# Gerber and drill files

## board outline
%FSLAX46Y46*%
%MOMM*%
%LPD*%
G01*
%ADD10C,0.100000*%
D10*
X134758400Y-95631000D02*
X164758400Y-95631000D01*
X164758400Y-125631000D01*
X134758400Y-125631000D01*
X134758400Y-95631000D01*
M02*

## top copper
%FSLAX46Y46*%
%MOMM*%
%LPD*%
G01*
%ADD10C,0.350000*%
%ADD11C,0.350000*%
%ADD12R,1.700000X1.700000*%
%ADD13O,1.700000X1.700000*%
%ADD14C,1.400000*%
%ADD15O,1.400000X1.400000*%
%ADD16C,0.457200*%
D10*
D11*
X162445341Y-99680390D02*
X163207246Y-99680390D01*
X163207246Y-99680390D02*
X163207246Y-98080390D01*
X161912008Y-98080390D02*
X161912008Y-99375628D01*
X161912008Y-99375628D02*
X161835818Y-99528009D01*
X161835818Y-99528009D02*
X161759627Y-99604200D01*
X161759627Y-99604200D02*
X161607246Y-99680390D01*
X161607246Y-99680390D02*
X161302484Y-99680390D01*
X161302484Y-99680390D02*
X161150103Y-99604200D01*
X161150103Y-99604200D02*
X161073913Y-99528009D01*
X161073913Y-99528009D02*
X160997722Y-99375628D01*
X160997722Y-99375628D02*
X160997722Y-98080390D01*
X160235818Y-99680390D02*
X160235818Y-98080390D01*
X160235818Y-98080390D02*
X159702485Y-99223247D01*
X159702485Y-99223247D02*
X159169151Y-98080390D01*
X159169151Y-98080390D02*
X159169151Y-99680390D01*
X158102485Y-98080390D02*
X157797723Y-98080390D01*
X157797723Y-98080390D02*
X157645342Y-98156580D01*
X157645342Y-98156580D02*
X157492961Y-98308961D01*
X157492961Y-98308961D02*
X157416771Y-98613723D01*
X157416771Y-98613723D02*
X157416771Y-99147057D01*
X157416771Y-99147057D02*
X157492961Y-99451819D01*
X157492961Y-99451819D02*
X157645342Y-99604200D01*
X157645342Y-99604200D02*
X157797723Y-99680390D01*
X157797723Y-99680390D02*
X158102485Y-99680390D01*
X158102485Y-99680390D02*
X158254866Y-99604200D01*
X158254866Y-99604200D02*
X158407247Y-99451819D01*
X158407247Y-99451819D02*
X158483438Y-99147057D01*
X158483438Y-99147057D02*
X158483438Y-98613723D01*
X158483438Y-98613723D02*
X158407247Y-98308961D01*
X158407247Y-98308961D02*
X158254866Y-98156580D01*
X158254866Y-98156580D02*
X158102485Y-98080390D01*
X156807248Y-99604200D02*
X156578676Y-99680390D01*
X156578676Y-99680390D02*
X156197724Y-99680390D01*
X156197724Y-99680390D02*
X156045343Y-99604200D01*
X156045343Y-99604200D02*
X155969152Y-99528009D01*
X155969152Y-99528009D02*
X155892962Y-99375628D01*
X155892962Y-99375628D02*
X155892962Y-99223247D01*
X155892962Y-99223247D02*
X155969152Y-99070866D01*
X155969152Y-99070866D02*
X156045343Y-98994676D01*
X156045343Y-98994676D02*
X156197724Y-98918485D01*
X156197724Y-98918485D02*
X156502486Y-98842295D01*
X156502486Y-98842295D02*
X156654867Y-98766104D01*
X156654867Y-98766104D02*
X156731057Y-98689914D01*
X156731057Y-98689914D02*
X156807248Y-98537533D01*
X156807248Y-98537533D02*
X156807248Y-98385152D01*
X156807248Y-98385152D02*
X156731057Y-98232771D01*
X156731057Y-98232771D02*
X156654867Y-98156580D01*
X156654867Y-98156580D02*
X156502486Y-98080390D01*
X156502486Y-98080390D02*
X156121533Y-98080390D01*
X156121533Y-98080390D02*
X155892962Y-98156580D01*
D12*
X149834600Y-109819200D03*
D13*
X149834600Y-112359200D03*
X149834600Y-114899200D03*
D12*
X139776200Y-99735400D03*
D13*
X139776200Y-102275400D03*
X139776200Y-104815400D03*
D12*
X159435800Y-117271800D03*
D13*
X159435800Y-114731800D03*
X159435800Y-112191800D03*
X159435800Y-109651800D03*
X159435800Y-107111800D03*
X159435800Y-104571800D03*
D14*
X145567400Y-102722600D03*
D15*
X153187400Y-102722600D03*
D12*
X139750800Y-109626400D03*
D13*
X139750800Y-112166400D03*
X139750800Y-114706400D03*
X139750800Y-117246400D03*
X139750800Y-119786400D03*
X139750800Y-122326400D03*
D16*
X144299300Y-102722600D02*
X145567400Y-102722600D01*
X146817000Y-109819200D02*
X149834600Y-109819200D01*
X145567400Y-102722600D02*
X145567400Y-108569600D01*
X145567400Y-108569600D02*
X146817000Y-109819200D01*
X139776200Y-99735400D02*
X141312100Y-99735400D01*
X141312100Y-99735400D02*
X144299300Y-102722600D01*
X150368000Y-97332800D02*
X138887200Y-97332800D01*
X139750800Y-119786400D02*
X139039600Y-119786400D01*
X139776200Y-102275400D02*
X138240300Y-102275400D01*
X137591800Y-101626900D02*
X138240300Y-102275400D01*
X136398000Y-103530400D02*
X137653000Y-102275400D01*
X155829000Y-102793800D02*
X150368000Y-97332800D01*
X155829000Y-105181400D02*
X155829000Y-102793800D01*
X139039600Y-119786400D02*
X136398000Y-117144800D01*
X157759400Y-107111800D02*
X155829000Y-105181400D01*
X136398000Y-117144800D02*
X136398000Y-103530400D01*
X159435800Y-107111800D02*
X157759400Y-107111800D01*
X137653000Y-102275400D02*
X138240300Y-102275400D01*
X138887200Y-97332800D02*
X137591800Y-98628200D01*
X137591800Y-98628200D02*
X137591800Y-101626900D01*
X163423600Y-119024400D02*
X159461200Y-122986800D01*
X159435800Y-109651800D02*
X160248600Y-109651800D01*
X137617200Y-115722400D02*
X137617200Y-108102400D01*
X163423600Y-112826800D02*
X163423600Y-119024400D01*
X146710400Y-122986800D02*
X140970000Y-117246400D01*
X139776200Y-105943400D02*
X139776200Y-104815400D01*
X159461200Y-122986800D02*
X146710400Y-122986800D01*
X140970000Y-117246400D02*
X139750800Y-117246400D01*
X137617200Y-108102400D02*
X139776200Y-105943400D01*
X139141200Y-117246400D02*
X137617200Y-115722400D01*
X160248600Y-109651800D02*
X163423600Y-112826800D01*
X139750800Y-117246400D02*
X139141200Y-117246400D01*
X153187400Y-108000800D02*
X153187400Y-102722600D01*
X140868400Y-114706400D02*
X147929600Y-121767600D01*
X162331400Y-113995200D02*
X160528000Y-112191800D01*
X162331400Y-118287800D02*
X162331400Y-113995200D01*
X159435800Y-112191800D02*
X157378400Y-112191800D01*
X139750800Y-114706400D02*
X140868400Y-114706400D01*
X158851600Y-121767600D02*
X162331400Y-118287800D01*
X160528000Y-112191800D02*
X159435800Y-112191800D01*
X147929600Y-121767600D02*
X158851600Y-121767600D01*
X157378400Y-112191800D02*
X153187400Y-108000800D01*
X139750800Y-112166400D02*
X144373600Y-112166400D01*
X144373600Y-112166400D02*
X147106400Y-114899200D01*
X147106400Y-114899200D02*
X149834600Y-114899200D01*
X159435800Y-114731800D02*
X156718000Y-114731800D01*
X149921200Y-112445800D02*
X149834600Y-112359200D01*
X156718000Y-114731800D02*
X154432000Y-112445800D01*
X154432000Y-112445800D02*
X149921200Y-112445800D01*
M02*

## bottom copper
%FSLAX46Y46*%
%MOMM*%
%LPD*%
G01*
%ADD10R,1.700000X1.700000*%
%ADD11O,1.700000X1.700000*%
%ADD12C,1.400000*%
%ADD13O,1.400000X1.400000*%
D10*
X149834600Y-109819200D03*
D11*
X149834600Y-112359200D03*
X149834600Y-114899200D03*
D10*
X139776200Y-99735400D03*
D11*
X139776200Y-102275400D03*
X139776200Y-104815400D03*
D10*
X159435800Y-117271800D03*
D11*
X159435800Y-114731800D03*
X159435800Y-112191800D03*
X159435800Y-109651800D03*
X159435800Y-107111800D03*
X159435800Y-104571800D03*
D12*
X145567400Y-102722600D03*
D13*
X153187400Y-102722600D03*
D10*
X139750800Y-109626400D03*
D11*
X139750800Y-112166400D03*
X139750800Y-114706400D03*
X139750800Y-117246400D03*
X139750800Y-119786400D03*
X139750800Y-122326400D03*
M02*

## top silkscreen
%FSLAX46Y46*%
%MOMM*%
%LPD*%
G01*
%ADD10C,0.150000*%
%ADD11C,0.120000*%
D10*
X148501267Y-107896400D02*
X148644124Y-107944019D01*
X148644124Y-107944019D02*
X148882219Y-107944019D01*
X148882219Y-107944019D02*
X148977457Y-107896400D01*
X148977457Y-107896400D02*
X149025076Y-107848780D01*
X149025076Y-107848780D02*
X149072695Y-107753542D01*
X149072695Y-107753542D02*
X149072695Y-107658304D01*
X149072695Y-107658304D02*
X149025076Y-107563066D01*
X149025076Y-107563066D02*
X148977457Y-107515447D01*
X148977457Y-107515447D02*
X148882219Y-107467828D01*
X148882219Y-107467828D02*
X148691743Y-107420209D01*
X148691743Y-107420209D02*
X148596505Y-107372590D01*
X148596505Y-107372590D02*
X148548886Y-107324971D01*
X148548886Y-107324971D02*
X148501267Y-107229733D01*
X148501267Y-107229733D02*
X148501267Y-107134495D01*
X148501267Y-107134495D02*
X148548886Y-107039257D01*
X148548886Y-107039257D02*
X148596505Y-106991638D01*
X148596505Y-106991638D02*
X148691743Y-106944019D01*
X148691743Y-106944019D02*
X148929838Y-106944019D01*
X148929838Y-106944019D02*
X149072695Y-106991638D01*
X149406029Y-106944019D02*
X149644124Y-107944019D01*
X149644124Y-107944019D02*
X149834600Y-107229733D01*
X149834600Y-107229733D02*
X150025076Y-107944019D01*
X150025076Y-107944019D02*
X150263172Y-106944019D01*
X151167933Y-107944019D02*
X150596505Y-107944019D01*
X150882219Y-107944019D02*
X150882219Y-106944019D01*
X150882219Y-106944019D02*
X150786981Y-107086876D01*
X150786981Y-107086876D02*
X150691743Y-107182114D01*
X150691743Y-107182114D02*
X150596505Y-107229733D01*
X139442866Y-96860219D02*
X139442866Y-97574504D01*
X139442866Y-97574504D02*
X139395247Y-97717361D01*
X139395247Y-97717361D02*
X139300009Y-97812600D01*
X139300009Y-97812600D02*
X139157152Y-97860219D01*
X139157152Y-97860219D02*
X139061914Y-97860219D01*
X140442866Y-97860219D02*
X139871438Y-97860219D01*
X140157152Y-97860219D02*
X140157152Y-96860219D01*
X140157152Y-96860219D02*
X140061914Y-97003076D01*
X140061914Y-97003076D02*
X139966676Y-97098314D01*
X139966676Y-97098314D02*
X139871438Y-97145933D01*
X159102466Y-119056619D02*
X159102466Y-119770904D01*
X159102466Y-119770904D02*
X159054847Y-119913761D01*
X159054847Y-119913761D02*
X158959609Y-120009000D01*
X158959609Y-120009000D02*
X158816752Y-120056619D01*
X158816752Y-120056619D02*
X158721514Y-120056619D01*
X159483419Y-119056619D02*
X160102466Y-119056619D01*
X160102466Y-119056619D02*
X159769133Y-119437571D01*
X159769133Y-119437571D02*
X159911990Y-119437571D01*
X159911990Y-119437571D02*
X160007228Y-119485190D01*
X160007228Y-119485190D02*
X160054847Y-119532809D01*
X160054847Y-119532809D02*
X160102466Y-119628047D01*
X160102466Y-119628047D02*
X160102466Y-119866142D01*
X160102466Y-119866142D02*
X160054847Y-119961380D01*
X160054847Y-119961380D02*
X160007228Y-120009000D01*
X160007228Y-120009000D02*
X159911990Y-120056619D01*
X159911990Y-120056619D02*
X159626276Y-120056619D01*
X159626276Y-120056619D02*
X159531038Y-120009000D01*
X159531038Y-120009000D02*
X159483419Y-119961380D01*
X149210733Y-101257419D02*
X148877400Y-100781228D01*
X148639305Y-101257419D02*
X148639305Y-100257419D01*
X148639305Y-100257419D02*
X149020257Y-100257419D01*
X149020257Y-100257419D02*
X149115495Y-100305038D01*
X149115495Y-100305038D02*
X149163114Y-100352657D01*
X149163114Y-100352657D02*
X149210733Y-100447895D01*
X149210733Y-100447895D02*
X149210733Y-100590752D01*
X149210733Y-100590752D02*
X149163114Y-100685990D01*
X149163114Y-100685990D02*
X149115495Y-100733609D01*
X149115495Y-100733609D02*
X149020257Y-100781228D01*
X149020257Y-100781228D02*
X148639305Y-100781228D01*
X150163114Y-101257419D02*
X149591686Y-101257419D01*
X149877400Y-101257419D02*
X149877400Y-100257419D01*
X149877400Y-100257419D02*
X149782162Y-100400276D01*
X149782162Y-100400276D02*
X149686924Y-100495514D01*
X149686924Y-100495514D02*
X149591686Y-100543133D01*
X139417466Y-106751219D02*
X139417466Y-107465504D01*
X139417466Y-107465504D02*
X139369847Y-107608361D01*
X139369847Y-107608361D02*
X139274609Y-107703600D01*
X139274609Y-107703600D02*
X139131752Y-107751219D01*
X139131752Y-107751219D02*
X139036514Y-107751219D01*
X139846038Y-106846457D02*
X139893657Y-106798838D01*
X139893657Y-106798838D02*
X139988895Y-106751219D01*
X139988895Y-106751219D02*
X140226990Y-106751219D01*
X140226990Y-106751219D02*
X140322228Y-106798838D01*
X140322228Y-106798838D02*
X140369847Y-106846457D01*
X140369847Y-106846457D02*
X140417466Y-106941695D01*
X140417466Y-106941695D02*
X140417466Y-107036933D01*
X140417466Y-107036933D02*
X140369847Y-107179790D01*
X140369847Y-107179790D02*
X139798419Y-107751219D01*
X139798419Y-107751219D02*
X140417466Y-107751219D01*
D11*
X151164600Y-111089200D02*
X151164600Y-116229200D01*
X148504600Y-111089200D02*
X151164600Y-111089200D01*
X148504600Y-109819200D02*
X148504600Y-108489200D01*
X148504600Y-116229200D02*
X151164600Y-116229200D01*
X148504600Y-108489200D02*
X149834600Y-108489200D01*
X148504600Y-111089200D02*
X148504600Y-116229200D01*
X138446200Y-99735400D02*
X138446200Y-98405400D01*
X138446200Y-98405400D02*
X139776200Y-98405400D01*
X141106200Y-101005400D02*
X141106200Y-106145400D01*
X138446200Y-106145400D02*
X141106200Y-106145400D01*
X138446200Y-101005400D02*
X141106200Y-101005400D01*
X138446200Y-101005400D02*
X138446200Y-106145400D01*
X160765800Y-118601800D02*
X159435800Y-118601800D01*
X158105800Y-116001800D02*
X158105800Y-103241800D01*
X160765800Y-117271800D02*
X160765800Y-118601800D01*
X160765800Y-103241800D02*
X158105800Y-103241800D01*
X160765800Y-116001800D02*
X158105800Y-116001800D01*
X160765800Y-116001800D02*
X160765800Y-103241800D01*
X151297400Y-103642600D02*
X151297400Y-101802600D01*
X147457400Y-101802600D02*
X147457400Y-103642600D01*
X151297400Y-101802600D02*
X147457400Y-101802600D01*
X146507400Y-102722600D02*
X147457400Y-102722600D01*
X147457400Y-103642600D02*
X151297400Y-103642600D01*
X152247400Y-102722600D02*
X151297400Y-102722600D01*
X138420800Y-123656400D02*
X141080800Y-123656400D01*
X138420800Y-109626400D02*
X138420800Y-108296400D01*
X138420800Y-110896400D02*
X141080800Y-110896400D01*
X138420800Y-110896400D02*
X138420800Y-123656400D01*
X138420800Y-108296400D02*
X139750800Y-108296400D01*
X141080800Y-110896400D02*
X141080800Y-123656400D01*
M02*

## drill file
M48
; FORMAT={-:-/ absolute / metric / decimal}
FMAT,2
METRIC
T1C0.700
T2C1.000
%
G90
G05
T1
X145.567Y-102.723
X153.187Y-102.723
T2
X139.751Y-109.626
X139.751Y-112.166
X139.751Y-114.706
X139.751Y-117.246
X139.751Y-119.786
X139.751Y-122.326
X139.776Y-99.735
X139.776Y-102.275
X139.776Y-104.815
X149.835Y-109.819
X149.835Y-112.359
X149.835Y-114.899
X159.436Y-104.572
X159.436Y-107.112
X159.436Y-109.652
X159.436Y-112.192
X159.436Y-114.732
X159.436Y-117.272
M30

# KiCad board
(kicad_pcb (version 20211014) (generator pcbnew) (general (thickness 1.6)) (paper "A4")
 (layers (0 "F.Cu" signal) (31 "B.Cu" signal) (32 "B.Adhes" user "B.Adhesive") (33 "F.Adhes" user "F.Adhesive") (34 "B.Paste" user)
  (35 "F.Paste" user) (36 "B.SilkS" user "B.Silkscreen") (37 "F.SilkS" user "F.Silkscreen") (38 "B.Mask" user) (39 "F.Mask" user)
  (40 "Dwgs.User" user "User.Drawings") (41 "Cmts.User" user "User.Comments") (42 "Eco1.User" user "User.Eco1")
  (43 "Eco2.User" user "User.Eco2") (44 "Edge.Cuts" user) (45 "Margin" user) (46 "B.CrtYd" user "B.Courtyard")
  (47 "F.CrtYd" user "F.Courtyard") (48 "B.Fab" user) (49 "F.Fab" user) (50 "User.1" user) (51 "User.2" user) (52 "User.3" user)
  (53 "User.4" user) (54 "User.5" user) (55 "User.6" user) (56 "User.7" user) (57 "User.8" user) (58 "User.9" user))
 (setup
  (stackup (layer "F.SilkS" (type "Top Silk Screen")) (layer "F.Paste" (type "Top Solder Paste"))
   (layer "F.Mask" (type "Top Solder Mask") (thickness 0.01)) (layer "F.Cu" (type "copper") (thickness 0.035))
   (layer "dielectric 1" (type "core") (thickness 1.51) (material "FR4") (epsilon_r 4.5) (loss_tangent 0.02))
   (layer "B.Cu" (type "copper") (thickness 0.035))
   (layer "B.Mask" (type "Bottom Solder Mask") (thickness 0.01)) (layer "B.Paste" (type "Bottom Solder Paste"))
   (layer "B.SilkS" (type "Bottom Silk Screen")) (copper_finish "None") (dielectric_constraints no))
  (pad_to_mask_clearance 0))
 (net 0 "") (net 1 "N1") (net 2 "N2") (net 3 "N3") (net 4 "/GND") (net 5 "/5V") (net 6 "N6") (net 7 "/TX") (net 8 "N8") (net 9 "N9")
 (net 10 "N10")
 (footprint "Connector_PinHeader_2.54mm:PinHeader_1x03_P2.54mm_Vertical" (layer "F.Cu") (at 149.8346 109.8192)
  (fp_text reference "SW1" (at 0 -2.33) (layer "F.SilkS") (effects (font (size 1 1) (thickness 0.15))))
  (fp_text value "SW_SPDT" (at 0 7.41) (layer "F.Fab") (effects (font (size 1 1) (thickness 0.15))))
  (fp_line (start 1.33 1.27) (end 1.33 6.41) (layer "F.SilkS") (width 0.12))
  (fp_line (start -1.33 1.27) (end 1.33 1.27) (layer "F.SilkS") (width 0.12))
  (fp_line (start -1.33 0) (end -1.33 -1.33) (layer "F.SilkS") (width 0.12))
  (fp_line (start -1.33 6.41) (end 1.33 6.41) (layer "F.SilkS") (width 0.12))
  (fp_line (start -1.33 -1.33) (end 0 -1.33) (layer "F.SilkS") (width 0.12))
  (fp_line (start -1.33 1.27) (end -1.33 6.41) (layer "F.SilkS") (width 0.12))
  (pad "1" thru_hole rect (at 0 0) (size 1.7 1.7) (drill 1) (layers *.Cu *.Mask) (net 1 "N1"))
  (pad "2" thru_hole oval (at 0 2.54) (size 1.7 1.7) (drill 1) (layers *.Cu *.Mask) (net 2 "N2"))
  (pad "3" thru_hole oval (at 0 5.08) (size 1.7 1.7) (drill 1) (layers *.Cu *.Mask) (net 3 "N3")))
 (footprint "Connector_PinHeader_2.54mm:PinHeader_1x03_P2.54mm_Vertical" (layer "F.Cu") (at 139.7762 99.7354)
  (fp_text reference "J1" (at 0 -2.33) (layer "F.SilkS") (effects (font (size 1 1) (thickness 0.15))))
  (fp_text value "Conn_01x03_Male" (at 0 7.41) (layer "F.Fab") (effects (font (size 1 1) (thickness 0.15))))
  (fp_line (start -1.33 0) (end -1.33 -1.33) (layer "F.SilkS") (width 0.12))
  (fp_line (start -1.33 -1.33) (end 0 -1.33) (layer "F.SilkS") (width 0.12))
  (fp_line (start 1.33 1.27) (end 1.33 6.41) (layer "F.SilkS") (width 0.12))
  (fp_line (start -1.33 6.41) (end 1.33 6.41) (layer "F.SilkS") (width 0.12))
  (fp_line (start -1.33 1.27) (end 1.33 1.27) (layer "F.SilkS") (width 0.12))
  (fp_line (start -1.33 1.27) (end -1.33 6.41) (layer "F.SilkS") (width 0.12))
  (pad "1" thru_hole rect (at 0 0) (size 1.7 1.7) (drill 1) (layers *.Cu *.Mask) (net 1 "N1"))
  (pad "2" thru_hole oval (at 0 2.54) (size 1.7 1.7) (drill 1) (layers *.Cu *.Mask) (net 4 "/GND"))
  (pad "3" thru_hole oval (at 0 5.08) (size 1.7 1.7) (drill 1) (layers *.Cu *.Mask) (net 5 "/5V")))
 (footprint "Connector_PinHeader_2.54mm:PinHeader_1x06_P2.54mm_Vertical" (layer "F.Cu") (at 159.4358 117.2718 180)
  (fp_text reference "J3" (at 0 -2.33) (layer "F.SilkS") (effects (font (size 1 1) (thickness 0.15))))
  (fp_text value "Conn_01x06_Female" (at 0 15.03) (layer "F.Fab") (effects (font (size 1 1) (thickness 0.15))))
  (fp_line (start -1.33 -1.33) (end 0 -1.33) (layer "F.SilkS") (width 0.12))
  (fp_line (start 1.33 1.27) (end 1.33 14.03) (layer "F.SilkS") (width 0.12))
  (fp_line (start -1.33 0) (end -1.33 -1.33) (layer "F.SilkS") (width 0.12))
  (fp_line (start -1.33 14.03) (end 1.33 14.03) (layer "F.SilkS") (width 0.12))
  (fp_line (start -1.33 1.27) (end 1.33 1.27) (layer "F.SilkS") (width 0.12))
  (fp_line (start -1.33 1.27) (end -1.33 14.03) (layer "F.SilkS") (width 0.12))
  (pad "1" thru_hole rect (at 0 0 180) (size 1.7 1.7) (drill 1) (layers *.Cu *.Mask) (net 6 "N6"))
  (pad "2" thru_hole oval (at 0 2.54 180) (size 1.7 1.7) (drill 1) (layers *.Cu *.Mask) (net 2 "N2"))
  (pad "3" thru_hole oval (at 0 5.08 180) (size 1.7 1.7) (drill 1) (layers *.Cu *.Mask) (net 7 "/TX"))
  (pad "4" thru_hole oval (at 0 7.62 180) (size 1.7 1.7) (drill 1) (layers *.Cu *.Mask) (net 5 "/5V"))
  (pad "5" thru_hole oval (at 0 10.16 180) (size 1.7 1.7) (drill 1) (layers *.Cu *.Mask) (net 4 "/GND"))
  (pad "6" thru_hole oval (at 0 12.7 180) (size 1.7 1.7) (drill 1) (layers *.Cu *.Mask) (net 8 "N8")))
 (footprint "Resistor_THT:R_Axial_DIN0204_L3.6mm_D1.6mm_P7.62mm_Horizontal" (layer "F.Cu") (at 145.5674 102.7226)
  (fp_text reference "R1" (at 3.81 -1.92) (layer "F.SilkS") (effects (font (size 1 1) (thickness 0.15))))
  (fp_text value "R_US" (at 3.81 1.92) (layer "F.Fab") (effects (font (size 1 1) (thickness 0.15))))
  (fp_line (start 5.73 0.92) (end 5.73 -0.92) (layer "F.SilkS") (width 0.12))
  (fp_line (start 1.89 -0.92) (end 1.89 0.92) (layer "F.SilkS") (width 0.12))
  (fp_line (start 5.73 -0.92) (end 1.89 -0.92) (layer "F.SilkS") (width 0.12))
  (fp_line (start 0.94 0) (end 1.89 0) (layer "F.SilkS") (width 0.12))
  (fp_line (start 1.89 0.92) (end 5.73 0.92) (layer "F.SilkS") (width 0.12))
  (fp_line (start 6.68 0) (end 5.73 0) (layer "F.SilkS") (width 0.12))
  (pad "1" thru_hole circle (at 0 0) (size 1.4 1.4) (drill 0.7) (layers *.Cu *.Mask) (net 1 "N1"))
  (pad "2" thru_hole oval (at 7.62 0) (size 1.4 1.4) (drill 0.7) (layers *.Cu *.Mask) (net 7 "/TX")))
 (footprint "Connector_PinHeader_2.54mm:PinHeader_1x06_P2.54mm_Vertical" (layer "F.Cu") (at 139.7508 109.6264)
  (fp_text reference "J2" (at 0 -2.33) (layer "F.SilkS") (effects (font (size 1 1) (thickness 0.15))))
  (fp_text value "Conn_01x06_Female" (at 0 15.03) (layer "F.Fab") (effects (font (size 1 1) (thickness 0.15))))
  (fp_line (start -1.33 14.03) (end 1.33 14.03) (layer "F.SilkS") (width 0.12))
  (fp_line (start -1.33 0) (end -1.33 -1.33) (layer "F.SilkS") (width 0.12))
  (fp_line (start -1.33 1.27) (end 1.33 1.27) (layer "F.SilkS") (width 0.12))
  (fp_line (start -1.33 1.27) (end -1.33 14.03) (layer "F.SilkS") (width 0.12))
  (fp_line (start -1.33 -1.33) (end 0 -1.33) (layer "F.SilkS") (width 0.12))
  (fp_line (start 1.33 1.27) (end 1.33 14.03) (layer "F.SilkS") (width 0.12))
  (pad "1" thru_hole rect (at 0 0) (size 1.7 1.7) (drill 1) (layers *.Cu *.Mask) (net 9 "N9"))
  (pad "2" thru_hole oval (at 0 2.54) (size 1.7 1.7) (drill 1) (layers *.Cu *.Mask) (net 3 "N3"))
  (pad "3" thru_hole oval (at 0 5.08) (size 1.7 1.7) (drill 1) (layers *.Cu *.Mask) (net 7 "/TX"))
  (pad "4" thru_hole oval (at 0 7.62) (size 1.7 1.7) (drill 1) (layers *.Cu *.Mask) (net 5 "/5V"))
  (pad "5" thru_hole oval (at 0 10.16) (size 1.7 1.7) (drill 1) (layers *.Cu *.Mask) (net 4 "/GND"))
  (pad "6" thru_hole oval (at 0 12.7) (size 1.7 1.7) (drill 1) (layers *.Cu *.Mask) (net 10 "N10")))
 (gr_rect (start 134.7584 95.631) (end 164.7584 125.631) (layer "Edge.Cuts") (width 0.1) (fill none))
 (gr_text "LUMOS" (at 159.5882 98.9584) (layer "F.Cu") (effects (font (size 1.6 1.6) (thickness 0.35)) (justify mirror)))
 (segment (start 144.2993 102.7226) (end 145.5674 102.7226) (width 0.4572) (layer "F.Cu") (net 1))
 (segment (start 146.817 109.8192) (end 149.8346 109.8192) (width 0.4572) (layer "F.Cu") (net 1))
 (segment (start 145.5674 102.7226) (end 145.5674 108.5696) (width 0.4572) (layer "F.Cu") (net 1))
 (segment (start 145.5674 108.5696) (end 146.817 109.8192) (width 0.4572) (layer "F.Cu") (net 1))
 (segment (start 139.7762 99.7354) (end 141.3121 99.7354) (width 0.4572) (layer "F.Cu") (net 1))
 (segment (start 141.3121 99.7354) (end 144.2993 102.7226) (width 0.4572) (layer "F.Cu") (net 1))
 (segment (start 150.368 97.3328) (end 138.8872 97.3328) (width 0.4572) (layer "F.Cu") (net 4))
 (segment (start 139.7508 119.7864) (end 139.0396 119.7864) (width 0.4572) (layer "F.Cu") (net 4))
 (segment (start 139.7762 102.2754) (end 138.2403 102.2754) (width 0.4572) (layer "F.Cu") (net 4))
 (segment (start 137.5918 101.6269) (end 138.2403 102.2754) (width 0.4572) (layer "F.Cu") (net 4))
 (segment (start 136.398 103.5304) (end 137.653 102.2754) (width 0.4572) (layer "F.Cu") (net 4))
 (segment (start 155.829 102.7938) (end 150.368 97.3328) (width 0.4572) (layer "F.Cu") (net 4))
 (segment (start 155.829 105.1814) (end 155.829 102.7938) (width 0.4572) (layer "F.Cu") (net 4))
 (segment (start 139.0396 119.7864) (end 136.398 117.1448) (width 0.4572) (layer "F.Cu") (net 4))
 (segment (start 157.7594 107.1118) (end 155.829 105.1814) (width 0.4572) (layer "F.Cu") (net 4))
 (segment (start 136.398 117.1448) (end 136.398 103.5304) (width 0.4572) (layer "F.Cu") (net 4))
 (segment (start 159.4358 107.1118) (end 157.7594 107.1118) (width 0.4572) (layer "F.Cu") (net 4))
 (segment (start 137.653 102.2754) (end 138.2403 102.2754) (width 0.4572) (layer "F.Cu") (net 4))
 (segment (start 138.8872 97.3328) (end 137.5918 98.6282) (width 0.4572) (layer "F.Cu") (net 4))
 (segment (start 137.5918 98.6282) (end 137.5918 101.6269) (width 0.4572) (layer "F.Cu") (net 4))
 (segment (start 163.4236 119.0244) (end 159.4612 122.9868) (width 0.4572) (layer "F.Cu") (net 5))
 (segment (start 159.4358 109.6518) (end 160.2486 109.6518) (width 0.4572) (layer "F.Cu") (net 5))
 (segment (start 137.6172 115.7224) (end 137.6172 108.1024) (width 0.4572) (layer "F.Cu") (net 5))
 (segment (start 163.4236 112.8268) (end 163.4236 119.0244) (width 0.4572) (layer "F.Cu") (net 5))
 (segment (start 146.7104 122.9868) (end 140.97 117.2464) (width 0.4572) (layer "F.Cu") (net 5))
 (segment (start 139.7762 105.9434) (end 139.7762 104.8154) (width 0.4572) (layer "F.Cu") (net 5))
 (segment (start 159.4612 122.9868) (end 146.7104 122.9868) (width 0.4572) (layer "F.Cu") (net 5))
 (segment (start 140.97 117.2464) (end 139.7508 117.2464) (width 0.4572) (layer "F.Cu") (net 5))
 (segment (start 137.6172 108.1024) (end 139.7762 105.9434) (width 0.4572) (layer "F.Cu") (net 5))
 (segment (start 139.1412 117.2464) (end 137.6172 115.7224) (width 0.4572) (layer "F.Cu") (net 5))
 (segment (start 160.2486 109.6518) (end 163.4236 112.8268) (width 0.4572) (layer "F.Cu") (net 5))
 (segment (start 139.7508 117.2464) (end 139.1412 117.2464) (width 0.4572) (layer "F.Cu") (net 5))
 (segment (start 153.1874 108.0008) (end 153.1874 102.7226) (width 0.4572) (layer "F.Cu") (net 7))
 (segment (start 140.8684 114.7064) (end 147.9296 121.7676) (width 0.4572) (layer "F.Cu") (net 7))
 (segment (start 162.3314 113.9952) (end 160.528 112.1918) (width 0.4572) (layer "F.Cu") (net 7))
 (segment (start 162.3314 118.2878) (end 162.3314 113.9952) (width 0.4572) (layer "F.Cu") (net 7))
 (segment (start 159.4358 112.1918) (end 157.3784 112.1918) (width 0.4572) (layer "F.Cu") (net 7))
 (segment (start 139.7508 114.7064) (end 140.8684 114.7064) (width 0.4572) (layer "F.Cu") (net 7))
 (segment (start 158.8516 121.7676) (end 162.3314 118.2878) (width 0.4572) (layer "F.Cu") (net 7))
 (segment (start 160.528 112.1918) (end 159.4358 112.1918) (width 0.4572) (layer "F.Cu") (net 7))
 (segment (start 147.9296 121.7676) (end 158.8516 121.7676) (width 0.4572) (layer "F.Cu") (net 7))
 (segment (start 157.3784 112.1918) (end 153.1874 108.0008) (width 0.4572) (layer "F.Cu") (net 7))
 (segment (start 139.7508 112.1664) (end 144.3736 112.1664) (width 0.4572) (layer "F.Cu") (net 3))
 (segment (start 144.3736 112.1664) (end 147.1064 114.8992) (width 0.4572) (layer "F.Cu") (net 3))
 (segment (start 147.1064 114.8992) (end 149.8346 114.8992) (width 0.4572) (layer "F.Cu") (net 3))
 (segment (start 159.4358 114.7318) (end 156.718 114.7318) (width 0.4572) (layer "F.Cu") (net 2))
 (segment (start 149.9212 112.4458) (end 149.8346 112.3592) (width 0.4572) (layer "F.Cu") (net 2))
 (segment (start 156.718 114.7318) (end 154.432 112.4458) (width 0.4572) (layer "F.Cu") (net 2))
 (segment (start 154.432 112.4458) (end 149.9212 112.4458) (width 0.4572) (layer "F.Cu") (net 2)))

